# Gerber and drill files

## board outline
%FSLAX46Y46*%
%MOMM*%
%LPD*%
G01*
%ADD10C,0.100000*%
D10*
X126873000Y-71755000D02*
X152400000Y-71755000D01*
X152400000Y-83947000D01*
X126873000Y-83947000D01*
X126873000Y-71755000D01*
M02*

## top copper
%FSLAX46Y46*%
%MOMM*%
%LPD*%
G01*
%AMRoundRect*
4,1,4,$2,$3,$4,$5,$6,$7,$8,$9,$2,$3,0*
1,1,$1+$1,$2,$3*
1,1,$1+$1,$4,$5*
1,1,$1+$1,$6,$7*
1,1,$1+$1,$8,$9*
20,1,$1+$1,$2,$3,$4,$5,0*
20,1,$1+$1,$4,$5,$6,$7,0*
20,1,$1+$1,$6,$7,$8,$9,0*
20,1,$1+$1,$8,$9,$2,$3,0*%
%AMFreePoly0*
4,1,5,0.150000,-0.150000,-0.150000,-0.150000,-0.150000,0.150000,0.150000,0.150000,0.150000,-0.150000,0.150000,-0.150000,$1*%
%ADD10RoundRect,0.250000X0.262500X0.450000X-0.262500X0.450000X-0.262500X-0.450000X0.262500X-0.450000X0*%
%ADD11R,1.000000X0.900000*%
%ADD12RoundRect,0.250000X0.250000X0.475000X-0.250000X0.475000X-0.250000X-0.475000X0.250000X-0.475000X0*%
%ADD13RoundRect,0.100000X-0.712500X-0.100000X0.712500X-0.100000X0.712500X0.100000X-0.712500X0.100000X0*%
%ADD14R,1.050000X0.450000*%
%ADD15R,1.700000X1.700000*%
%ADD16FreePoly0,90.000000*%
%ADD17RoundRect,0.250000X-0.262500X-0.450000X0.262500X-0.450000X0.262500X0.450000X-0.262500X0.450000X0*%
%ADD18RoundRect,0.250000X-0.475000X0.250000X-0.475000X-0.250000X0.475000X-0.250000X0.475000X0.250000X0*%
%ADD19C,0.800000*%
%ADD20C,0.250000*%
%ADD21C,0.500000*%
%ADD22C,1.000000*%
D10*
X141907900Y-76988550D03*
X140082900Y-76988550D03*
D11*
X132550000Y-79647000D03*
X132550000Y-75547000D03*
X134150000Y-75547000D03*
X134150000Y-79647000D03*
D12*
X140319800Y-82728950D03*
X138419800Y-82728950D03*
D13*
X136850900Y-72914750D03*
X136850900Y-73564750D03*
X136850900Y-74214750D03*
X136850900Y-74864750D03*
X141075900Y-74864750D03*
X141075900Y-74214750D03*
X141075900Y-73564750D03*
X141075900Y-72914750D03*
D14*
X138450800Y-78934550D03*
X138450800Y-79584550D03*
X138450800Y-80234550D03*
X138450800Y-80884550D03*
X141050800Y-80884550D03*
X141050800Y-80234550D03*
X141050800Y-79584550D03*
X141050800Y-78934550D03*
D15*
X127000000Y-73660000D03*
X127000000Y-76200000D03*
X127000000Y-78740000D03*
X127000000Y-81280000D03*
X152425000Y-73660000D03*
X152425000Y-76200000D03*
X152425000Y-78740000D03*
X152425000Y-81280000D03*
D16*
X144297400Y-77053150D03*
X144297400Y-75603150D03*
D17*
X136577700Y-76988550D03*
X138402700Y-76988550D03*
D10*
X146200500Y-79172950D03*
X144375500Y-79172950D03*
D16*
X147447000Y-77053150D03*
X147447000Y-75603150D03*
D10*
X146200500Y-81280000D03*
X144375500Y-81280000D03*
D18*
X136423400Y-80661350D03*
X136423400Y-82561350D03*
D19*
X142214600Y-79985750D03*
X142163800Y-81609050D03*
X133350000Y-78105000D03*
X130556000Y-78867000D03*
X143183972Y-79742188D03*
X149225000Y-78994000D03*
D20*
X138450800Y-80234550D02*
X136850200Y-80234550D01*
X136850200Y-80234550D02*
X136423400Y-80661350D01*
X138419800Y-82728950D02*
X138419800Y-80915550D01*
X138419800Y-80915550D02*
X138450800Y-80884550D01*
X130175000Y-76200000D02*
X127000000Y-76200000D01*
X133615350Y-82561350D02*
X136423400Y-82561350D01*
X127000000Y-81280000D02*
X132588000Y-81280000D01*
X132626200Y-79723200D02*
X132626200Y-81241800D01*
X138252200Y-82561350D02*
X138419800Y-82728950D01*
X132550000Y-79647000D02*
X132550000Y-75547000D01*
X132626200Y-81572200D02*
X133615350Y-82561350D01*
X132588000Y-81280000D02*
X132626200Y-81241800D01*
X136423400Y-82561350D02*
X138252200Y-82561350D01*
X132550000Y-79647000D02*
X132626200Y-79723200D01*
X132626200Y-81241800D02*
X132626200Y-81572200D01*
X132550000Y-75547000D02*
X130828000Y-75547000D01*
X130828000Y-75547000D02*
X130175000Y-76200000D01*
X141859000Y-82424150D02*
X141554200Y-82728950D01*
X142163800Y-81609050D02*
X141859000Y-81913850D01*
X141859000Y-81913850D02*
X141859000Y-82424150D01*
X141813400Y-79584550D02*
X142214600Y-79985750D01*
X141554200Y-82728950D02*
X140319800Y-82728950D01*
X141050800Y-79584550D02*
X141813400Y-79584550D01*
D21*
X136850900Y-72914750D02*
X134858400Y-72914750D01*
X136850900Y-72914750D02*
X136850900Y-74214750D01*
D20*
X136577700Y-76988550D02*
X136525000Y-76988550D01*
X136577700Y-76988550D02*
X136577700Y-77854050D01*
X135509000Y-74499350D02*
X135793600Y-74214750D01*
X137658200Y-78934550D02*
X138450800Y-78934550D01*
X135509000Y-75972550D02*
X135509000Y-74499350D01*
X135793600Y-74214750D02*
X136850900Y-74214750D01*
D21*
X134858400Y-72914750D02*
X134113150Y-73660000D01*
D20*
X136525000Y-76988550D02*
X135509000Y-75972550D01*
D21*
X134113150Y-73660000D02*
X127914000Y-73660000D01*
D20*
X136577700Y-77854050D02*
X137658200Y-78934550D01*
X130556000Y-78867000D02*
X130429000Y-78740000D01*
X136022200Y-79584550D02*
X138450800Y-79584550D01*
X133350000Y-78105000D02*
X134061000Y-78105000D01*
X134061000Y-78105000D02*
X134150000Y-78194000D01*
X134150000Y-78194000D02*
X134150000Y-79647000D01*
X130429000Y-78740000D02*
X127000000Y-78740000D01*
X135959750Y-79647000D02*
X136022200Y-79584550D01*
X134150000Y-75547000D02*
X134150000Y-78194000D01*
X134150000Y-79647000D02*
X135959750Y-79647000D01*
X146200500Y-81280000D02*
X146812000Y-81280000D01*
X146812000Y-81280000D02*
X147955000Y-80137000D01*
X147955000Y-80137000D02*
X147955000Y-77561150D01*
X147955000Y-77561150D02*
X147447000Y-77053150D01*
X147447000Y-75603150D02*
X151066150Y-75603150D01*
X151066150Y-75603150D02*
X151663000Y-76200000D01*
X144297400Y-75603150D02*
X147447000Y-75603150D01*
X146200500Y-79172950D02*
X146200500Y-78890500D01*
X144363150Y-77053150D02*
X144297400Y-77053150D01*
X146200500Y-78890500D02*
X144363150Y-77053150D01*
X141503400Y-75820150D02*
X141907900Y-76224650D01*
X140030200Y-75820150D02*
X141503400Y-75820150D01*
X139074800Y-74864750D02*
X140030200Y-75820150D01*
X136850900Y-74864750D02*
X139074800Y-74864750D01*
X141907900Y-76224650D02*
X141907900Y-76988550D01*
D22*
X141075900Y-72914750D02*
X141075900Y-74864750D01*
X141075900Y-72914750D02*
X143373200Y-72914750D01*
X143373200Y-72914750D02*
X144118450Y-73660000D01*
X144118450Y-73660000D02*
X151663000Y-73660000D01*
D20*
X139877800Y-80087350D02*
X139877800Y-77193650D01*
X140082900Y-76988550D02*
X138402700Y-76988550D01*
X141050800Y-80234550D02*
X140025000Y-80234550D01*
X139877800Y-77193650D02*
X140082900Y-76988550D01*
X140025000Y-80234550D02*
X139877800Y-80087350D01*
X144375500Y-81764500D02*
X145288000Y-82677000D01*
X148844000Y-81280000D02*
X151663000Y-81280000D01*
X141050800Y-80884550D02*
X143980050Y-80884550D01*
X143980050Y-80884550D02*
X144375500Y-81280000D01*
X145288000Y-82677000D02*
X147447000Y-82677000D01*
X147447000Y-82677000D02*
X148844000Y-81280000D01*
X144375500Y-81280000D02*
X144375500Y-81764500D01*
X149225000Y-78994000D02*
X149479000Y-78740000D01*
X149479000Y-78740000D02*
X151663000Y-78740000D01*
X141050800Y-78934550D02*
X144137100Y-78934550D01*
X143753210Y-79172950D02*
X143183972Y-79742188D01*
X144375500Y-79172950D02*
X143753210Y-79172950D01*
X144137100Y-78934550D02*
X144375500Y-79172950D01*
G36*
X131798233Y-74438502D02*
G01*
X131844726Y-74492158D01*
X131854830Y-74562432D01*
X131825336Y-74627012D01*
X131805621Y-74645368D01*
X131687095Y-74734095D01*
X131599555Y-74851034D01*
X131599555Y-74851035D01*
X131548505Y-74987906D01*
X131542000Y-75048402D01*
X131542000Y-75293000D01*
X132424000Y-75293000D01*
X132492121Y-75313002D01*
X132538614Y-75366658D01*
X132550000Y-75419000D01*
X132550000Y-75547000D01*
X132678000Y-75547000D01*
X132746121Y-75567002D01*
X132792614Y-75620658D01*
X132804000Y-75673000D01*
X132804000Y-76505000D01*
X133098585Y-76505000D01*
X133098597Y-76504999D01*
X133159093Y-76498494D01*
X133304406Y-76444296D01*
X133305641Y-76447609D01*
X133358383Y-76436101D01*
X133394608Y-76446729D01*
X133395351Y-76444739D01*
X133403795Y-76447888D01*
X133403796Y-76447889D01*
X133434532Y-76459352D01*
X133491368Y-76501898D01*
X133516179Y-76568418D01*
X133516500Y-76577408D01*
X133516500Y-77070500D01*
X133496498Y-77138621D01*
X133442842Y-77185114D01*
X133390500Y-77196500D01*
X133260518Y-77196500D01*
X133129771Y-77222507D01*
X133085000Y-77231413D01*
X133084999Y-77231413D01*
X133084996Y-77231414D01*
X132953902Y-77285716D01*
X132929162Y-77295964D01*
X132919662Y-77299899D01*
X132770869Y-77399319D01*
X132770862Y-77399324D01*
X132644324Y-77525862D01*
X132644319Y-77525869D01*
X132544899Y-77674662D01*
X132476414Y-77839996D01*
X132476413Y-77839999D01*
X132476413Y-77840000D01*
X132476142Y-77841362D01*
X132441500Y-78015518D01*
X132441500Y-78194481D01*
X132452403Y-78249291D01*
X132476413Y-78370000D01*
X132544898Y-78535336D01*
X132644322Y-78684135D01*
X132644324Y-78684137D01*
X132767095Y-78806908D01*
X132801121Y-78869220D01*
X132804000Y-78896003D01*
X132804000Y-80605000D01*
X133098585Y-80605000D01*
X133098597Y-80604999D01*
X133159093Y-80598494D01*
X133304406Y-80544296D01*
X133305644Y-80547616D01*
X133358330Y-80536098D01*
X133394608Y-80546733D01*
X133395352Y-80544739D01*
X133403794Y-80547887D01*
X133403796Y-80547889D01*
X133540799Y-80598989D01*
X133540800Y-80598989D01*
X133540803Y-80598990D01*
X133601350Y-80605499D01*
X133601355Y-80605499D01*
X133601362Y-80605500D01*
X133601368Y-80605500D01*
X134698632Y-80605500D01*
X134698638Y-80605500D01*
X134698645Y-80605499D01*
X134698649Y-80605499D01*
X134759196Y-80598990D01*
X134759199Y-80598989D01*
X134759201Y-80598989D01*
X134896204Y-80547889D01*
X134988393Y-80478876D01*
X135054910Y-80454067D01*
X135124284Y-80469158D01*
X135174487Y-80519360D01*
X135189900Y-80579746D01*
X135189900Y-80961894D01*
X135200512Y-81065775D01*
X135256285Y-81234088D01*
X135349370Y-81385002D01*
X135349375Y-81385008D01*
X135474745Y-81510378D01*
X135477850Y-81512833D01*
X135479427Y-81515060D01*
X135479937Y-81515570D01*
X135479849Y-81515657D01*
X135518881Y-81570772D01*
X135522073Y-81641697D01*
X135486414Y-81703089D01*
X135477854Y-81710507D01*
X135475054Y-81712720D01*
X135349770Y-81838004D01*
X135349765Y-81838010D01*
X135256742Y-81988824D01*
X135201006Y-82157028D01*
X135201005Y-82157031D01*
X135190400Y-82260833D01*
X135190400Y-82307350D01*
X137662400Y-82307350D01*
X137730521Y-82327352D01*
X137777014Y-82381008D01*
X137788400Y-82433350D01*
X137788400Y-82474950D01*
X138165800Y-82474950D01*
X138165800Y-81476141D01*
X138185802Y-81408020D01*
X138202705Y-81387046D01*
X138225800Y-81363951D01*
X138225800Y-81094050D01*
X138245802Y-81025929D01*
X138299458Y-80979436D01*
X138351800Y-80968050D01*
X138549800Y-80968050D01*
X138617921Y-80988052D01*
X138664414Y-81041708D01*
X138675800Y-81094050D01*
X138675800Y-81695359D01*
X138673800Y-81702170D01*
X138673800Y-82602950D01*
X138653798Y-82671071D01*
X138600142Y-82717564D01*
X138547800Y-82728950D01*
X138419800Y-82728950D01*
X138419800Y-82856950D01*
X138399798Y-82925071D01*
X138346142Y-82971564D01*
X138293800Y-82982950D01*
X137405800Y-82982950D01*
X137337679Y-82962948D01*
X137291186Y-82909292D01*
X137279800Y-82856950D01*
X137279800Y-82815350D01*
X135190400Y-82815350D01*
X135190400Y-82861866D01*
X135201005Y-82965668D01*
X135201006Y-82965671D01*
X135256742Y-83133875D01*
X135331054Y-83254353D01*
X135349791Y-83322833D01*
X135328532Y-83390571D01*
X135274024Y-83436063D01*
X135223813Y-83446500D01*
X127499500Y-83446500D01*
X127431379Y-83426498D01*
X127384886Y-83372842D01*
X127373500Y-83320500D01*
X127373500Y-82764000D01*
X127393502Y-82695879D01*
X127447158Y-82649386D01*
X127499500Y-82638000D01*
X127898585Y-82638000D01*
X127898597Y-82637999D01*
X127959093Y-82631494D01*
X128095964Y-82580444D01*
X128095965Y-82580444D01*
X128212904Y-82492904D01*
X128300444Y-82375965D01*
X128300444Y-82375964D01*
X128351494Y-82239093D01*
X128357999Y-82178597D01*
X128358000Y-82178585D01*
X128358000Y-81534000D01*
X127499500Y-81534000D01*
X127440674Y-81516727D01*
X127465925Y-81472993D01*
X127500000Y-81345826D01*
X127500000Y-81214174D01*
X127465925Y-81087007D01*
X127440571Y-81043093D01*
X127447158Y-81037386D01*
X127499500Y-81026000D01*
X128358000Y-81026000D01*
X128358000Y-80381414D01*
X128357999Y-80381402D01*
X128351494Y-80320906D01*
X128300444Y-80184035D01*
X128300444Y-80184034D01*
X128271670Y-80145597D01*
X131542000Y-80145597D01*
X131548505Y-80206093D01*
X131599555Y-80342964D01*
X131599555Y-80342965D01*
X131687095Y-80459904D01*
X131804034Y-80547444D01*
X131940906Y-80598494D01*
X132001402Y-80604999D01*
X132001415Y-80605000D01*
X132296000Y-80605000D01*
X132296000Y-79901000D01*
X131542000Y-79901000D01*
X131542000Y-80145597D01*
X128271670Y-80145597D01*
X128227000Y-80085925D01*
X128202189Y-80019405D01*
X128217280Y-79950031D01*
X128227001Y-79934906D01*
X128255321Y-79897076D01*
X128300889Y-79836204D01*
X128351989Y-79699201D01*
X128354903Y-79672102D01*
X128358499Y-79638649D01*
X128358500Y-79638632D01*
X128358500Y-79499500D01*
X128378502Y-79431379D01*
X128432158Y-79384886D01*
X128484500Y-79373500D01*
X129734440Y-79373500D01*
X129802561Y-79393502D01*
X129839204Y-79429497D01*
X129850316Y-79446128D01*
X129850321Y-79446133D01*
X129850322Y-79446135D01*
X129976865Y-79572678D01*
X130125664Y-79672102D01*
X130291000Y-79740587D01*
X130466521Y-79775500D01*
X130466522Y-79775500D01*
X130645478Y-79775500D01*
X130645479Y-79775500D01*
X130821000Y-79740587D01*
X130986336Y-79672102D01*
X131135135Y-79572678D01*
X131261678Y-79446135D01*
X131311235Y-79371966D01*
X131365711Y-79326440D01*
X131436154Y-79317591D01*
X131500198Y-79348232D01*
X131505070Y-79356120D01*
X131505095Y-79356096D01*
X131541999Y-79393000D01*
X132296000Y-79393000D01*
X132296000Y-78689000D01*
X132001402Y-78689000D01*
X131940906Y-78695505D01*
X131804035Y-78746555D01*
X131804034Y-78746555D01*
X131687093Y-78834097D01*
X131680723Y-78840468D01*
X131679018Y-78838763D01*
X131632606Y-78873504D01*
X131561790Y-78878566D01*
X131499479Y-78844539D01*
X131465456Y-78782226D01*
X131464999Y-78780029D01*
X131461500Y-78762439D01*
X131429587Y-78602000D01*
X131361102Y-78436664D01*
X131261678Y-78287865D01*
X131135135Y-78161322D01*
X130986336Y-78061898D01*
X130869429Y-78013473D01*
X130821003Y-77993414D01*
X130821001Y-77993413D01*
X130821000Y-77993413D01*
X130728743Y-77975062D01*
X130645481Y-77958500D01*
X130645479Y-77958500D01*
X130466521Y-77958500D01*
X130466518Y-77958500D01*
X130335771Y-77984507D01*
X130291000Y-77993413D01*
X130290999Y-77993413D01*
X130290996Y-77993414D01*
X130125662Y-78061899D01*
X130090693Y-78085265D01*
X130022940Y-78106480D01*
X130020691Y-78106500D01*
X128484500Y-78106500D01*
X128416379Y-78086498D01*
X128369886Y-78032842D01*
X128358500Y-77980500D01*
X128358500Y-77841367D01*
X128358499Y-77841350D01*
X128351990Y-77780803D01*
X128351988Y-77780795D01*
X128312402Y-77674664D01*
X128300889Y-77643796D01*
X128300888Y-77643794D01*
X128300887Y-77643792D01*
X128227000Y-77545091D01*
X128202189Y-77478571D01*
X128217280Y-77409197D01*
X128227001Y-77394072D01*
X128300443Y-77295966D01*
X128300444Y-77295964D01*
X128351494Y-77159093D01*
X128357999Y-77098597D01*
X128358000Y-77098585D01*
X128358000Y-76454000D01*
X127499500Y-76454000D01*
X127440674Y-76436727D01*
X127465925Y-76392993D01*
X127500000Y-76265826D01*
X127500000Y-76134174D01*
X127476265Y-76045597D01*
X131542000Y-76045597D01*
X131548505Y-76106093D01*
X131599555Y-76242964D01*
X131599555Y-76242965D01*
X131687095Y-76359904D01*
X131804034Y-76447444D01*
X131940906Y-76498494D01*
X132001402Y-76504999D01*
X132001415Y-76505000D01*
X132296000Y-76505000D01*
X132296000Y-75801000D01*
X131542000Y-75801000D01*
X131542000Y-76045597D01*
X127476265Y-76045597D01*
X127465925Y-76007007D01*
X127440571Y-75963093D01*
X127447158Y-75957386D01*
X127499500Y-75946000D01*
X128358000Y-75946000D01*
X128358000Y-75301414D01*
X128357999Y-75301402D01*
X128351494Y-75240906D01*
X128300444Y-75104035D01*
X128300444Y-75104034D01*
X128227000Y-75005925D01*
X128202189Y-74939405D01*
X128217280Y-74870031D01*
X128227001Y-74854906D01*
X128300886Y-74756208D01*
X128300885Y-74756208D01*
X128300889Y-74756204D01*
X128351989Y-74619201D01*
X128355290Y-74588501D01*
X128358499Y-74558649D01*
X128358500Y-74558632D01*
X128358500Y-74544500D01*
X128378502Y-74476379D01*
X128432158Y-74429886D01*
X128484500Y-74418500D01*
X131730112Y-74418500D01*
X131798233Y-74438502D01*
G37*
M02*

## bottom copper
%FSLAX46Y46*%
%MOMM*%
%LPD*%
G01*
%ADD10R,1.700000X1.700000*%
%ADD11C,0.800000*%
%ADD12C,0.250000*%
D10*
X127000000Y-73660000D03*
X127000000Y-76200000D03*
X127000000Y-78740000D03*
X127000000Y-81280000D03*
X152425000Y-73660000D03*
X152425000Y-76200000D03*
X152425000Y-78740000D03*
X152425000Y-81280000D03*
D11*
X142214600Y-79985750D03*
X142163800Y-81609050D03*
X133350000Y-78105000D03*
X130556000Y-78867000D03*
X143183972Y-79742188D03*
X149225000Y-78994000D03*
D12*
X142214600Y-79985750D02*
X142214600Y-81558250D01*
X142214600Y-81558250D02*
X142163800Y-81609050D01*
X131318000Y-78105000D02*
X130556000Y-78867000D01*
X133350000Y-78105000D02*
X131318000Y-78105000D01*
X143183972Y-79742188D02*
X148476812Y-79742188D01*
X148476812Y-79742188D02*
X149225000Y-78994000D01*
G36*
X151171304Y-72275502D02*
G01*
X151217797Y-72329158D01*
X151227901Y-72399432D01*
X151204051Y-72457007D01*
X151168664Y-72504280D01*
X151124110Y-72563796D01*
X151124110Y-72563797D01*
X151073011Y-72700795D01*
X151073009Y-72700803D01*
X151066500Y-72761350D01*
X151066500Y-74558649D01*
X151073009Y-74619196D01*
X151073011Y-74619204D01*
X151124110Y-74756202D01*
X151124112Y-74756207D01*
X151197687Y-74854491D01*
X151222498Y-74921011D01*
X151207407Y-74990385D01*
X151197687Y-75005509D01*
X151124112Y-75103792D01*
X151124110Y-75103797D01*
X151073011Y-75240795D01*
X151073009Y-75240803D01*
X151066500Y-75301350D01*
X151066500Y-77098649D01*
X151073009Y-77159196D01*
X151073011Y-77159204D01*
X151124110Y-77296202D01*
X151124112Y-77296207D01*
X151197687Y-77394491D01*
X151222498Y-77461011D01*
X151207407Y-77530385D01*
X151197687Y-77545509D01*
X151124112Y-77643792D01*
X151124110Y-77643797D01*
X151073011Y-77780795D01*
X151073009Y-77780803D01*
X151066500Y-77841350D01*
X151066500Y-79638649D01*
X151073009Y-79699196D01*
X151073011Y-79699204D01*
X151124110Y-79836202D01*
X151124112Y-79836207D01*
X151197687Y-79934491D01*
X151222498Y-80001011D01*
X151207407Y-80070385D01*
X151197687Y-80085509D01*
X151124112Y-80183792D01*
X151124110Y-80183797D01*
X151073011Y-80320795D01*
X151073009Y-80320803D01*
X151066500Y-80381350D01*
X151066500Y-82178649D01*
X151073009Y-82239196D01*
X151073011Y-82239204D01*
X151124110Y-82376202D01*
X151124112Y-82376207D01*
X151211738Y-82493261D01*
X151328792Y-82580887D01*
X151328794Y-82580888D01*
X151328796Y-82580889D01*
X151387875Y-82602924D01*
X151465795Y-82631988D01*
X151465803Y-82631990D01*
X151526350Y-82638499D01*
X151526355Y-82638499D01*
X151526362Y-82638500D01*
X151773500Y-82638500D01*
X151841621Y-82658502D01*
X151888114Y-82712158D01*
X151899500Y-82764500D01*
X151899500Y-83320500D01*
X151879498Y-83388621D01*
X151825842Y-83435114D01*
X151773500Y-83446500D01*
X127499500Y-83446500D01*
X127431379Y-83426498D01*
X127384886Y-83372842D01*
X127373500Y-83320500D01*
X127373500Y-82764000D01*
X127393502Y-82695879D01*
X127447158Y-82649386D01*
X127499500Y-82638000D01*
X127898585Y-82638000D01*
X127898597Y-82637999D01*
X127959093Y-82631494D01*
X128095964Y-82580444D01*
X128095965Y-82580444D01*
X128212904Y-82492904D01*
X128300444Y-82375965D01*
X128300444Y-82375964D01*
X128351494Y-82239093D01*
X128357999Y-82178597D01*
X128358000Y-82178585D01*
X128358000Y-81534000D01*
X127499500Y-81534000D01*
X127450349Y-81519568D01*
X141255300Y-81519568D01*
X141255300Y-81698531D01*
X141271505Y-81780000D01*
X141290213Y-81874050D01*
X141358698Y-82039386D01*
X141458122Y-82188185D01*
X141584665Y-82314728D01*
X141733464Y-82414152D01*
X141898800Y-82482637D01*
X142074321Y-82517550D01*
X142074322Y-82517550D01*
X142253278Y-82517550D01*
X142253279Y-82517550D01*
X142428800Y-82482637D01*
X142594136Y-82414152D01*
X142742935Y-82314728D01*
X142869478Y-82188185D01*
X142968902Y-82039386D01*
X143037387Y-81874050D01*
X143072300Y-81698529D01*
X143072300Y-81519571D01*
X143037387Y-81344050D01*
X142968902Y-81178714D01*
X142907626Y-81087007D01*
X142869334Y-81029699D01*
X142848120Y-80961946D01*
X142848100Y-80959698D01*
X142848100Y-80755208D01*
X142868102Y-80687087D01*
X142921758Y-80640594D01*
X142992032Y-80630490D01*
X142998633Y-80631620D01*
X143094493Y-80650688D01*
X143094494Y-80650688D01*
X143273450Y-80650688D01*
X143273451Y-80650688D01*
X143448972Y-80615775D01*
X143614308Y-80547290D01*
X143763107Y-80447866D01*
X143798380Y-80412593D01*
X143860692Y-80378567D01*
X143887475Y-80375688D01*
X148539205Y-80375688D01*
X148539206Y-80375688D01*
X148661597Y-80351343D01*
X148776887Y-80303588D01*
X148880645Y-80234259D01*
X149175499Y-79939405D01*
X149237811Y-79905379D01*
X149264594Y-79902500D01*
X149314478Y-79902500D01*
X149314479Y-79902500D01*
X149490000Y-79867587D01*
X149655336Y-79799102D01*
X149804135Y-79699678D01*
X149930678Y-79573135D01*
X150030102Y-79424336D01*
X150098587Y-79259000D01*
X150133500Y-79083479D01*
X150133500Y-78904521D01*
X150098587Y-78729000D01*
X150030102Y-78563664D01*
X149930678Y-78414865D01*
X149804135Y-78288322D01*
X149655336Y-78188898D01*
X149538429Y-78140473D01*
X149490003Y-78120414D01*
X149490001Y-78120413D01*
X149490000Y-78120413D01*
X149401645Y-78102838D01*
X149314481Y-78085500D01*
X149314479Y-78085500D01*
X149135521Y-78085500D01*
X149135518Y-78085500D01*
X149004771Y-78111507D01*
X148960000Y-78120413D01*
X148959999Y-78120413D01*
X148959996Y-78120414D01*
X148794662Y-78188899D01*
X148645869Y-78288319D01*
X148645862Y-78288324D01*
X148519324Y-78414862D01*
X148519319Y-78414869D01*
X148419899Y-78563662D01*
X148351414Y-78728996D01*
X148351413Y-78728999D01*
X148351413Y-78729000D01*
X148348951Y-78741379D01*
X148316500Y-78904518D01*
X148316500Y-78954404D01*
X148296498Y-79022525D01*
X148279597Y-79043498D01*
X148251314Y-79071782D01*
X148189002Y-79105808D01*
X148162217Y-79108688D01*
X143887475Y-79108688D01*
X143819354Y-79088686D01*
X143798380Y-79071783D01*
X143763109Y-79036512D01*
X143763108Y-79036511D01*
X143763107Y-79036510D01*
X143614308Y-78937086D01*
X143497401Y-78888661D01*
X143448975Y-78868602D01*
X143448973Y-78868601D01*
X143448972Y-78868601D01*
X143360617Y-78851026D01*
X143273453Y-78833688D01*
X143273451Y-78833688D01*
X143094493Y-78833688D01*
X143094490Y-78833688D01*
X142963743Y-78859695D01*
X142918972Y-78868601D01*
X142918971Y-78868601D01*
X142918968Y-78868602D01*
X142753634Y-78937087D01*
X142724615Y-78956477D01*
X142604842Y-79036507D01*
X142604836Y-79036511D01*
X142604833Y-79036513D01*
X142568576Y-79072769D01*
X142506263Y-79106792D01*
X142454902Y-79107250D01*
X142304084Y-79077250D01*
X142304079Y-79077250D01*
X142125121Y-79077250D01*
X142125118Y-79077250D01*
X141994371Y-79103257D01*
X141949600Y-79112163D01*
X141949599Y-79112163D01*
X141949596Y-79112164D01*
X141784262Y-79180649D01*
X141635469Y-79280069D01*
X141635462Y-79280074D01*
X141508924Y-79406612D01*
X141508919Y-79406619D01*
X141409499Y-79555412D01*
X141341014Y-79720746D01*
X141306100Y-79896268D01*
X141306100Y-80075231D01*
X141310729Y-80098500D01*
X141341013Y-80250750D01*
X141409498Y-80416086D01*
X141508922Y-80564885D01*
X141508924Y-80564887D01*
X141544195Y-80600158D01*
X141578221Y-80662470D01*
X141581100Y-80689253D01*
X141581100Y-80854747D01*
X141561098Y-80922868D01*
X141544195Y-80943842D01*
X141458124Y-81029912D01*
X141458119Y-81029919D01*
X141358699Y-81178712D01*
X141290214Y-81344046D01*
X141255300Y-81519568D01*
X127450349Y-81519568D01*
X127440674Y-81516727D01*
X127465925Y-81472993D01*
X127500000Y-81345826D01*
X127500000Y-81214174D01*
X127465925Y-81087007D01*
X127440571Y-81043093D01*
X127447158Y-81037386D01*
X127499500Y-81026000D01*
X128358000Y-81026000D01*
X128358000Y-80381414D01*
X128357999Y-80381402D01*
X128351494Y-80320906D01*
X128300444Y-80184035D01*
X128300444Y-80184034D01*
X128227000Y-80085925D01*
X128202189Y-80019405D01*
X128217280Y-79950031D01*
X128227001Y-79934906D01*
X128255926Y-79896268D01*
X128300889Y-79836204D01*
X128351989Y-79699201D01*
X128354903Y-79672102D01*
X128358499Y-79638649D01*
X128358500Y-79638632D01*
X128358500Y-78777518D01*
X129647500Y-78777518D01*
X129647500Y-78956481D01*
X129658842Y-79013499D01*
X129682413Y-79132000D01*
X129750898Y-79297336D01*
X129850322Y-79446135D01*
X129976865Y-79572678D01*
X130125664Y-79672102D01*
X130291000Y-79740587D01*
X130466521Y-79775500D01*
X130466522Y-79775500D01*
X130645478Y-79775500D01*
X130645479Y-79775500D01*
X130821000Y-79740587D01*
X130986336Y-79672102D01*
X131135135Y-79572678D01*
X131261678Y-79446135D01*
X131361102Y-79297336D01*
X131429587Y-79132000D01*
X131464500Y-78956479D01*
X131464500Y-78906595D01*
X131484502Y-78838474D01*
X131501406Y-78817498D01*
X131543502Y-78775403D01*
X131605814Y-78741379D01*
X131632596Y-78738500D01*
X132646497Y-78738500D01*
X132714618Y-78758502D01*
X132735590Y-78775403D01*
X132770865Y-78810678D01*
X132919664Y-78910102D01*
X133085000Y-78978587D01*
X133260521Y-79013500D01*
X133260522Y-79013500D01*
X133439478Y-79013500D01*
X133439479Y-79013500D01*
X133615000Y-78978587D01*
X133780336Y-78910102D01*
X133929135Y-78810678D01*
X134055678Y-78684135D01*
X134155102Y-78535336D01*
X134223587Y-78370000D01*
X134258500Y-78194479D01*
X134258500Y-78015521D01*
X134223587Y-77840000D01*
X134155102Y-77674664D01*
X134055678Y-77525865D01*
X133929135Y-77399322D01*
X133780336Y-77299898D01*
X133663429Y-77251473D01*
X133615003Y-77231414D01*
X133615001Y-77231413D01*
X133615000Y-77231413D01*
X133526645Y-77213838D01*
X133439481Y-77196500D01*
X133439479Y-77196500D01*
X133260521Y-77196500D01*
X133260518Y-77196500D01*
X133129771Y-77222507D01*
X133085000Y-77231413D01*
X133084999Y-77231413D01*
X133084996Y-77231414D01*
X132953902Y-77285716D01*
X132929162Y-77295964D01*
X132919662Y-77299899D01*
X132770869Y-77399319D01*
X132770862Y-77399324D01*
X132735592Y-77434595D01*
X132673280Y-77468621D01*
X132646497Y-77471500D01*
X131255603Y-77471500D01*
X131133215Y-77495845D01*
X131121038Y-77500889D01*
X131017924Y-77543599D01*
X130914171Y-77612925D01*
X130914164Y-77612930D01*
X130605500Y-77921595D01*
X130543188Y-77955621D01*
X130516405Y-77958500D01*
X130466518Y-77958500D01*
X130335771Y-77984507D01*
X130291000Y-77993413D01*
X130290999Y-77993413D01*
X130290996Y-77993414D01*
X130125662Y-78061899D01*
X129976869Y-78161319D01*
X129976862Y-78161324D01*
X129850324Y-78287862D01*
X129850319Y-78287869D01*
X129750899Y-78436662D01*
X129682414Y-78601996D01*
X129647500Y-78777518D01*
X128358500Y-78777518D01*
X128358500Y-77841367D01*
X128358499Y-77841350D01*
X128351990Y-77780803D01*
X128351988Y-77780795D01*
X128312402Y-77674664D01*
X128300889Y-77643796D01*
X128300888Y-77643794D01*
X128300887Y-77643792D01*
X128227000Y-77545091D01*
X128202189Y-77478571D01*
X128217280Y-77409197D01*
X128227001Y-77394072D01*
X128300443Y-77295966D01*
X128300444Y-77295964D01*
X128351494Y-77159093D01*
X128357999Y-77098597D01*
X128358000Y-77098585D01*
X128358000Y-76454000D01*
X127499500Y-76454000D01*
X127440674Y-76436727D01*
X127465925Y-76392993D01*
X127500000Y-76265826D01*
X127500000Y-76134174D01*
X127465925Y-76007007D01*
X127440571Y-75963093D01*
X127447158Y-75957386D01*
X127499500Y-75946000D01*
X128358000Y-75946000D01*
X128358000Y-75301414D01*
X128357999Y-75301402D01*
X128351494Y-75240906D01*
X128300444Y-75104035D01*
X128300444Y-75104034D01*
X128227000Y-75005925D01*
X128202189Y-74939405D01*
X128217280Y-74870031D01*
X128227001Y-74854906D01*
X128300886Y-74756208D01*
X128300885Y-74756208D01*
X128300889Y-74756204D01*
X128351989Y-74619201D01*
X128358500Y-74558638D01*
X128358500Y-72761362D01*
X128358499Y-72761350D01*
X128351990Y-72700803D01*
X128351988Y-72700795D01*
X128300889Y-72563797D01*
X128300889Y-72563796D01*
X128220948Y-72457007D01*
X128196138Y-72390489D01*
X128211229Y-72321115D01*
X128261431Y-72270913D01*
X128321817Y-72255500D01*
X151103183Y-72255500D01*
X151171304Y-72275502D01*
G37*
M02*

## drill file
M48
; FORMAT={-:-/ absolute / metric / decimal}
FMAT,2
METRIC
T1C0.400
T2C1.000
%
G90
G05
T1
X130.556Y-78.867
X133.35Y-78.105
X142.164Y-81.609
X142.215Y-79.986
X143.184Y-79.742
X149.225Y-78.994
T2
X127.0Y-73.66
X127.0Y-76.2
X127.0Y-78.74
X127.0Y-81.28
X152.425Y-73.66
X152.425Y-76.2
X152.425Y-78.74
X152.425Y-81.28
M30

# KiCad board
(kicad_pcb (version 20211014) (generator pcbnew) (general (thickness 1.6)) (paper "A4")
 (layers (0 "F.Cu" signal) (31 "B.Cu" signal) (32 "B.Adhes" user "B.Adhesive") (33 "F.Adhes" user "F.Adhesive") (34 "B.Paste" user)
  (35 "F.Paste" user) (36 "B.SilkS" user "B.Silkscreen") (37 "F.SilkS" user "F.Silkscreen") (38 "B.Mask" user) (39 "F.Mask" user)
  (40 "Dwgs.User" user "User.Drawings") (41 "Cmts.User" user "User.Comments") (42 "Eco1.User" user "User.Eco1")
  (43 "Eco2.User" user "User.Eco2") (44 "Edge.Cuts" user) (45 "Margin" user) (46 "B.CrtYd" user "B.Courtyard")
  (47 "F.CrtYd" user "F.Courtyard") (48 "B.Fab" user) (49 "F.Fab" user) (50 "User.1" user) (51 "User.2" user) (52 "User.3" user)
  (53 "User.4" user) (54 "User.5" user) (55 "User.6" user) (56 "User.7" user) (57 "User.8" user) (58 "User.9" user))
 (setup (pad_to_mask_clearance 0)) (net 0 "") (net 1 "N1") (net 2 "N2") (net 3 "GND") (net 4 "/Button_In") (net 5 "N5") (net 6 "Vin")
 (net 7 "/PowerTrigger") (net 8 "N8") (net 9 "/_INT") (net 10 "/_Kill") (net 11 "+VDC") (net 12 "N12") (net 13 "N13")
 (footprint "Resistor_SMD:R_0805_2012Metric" (layer "F.Cu") (at 140.9954 76.98855 180)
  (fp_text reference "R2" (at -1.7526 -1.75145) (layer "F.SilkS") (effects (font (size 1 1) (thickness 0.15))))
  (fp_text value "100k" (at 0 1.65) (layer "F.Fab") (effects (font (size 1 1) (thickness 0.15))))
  (pad "1" smd roundrect locked (at -0.9125 0 180) (size 1.025 1.4) (layers "F.Cu" "F.Paste" "F.Mask") (roundrect_rratio 0.243902)
   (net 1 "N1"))
  (pad "2" smd roundrect locked (at 0.9125 0 180) (size 1.025 1.4) (layers "F.Cu" "F.Paste" "F.Mask") (roundrect_rratio 0.243902)
   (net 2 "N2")))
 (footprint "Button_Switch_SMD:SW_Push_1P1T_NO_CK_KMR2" (layer "F.Cu") (at 133.35 77.597 90)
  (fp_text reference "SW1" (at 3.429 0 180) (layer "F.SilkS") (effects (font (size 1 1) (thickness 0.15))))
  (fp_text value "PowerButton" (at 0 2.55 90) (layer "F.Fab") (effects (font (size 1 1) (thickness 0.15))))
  (pad "1" smd rect locked (at -2.05 -0.8 90) (size 0.9 1) (layers "F.Cu" "F.Paste" "F.Mask") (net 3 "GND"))
  (pad "1" smd rect locked (at 2.05 -0.8 90) (size 0.9 1) (layers "F.Cu" "F.Paste" "F.Mask") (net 3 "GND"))
  (pad "2" smd rect locked (at 2.05 0.8 90) (size 0.9 1) (layers "F.Cu" "F.Paste" "F.Mask") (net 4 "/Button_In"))
  (pad "2" smd rect locked (at -2.05 0.8 90) (size 0.9 1) (layers "F.Cu" "F.Paste" "F.Mask") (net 4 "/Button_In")))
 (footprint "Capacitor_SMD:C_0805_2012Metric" (layer "F.Cu") (at 139.3698 82.72895 180)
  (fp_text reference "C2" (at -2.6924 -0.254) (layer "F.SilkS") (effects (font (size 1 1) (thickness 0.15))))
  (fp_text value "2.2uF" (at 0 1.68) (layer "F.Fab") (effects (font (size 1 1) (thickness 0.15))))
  (pad "1" smd roundrect locked (at -0.95 0 180) (size 1 1.45) (layers "F.Cu" "F.Paste" "F.Mask") (roundrect_rratio 0.25) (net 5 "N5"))
  (pad "2" smd roundrect locked (at 0.95 0 180) (size 1 1.45) (layers "F.Cu" "F.Paste" "F.Mask") (roundrect_rratio 0.25) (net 3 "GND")))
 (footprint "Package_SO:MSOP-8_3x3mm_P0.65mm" (layer "F.Cu") (at 138.9634 73.88975)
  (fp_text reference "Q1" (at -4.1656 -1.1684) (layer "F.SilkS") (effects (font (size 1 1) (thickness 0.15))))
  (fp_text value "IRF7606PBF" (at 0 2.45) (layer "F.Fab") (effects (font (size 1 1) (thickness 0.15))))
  (pad "1" smd roundrect locked (at -2.1125 -0.975) (size 1.625 0.4) (layers "F.Cu" "F.Paste" "F.Mask") (roundrect_rratio 0.25)
   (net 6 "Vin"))
  (pad "2" smd roundrect locked (at -2.1125 -0.325) (size 1.625 0.4) (layers "F.Cu" "F.Paste" "F.Mask") (roundrect_rratio 0.25)
   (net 6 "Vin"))
  (pad "3" smd roundrect locked (at -2.1125 0.325) (size 1.625 0.4) (layers "F.Cu" "F.Paste" "F.Mask") (roundrect_rratio 0.25) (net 6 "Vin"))
  (pad "4" smd roundrect locked (at -2.1125 0.975) (size 1.625 0.4) (layers "F.Cu" "F.Paste" "F.Mask") (roundrect_rratio 0.25) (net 1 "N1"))
  (pad "5" smd roundrect locked (at 2.1125 0.975) (size 1.625 0.4) (layers "F.Cu" "F.Paste" "F.Mask") (roundrect_rratio 0.25)
   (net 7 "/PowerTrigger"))
  (pad "6" smd roundrect locked (at 2.1125 0.325) (size 1.625 0.4) (layers "F.Cu" "F.Paste" "F.Mask") (roundrect_rratio 0.25)
   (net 7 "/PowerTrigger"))
  (pad "7" smd roundrect locked (at 2.1125 -0.325) (size 1.625 0.4) (layers "F.Cu" "F.Paste" "F.Mask") (roundrect_rratio 0.25)
   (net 7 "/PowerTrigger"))
  (pad "8" smd roundrect locked (at 2.1125 -0.975) (size 1.625 0.4) (layers "F.Cu" "F.Paste" "F.Mask") (roundrect_rratio 0.25)
   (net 7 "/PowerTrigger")))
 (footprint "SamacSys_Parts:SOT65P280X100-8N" (layer "F.Cu") (at 139.7508 79.90955)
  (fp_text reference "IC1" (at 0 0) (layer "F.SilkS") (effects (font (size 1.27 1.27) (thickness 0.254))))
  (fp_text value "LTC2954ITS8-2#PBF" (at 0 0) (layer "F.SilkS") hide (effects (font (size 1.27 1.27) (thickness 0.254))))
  (pad "1" smd rect locked (at -1.3 -0.975 90) (size 0.45 1.05) (layers "F.Cu" "F.Paste" "F.Mask") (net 6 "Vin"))
  (pad "2" smd rect locked (at -1.3 -0.325 90) (size 0.45 1.05) (layers "F.Cu" "F.Paste" "F.Mask") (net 4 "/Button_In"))
  (pad "3" smd rect locked (at -1.3 0.325 90) (size 0.45 1.05) (layers "F.Cu" "F.Paste" "F.Mask") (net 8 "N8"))
  (pad "4" smd rect locked (at -1.3 0.975 90) (size 0.45 1.05) (layers "F.Cu" "F.Paste" "F.Mask") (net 3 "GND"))
  (pad "5" smd rect locked (at 1.3 0.975 90) (size 0.45 1.05) (layers "F.Cu" "F.Paste" "F.Mask") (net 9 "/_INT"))
  (pad "6" smd rect locked (at 1.3 0.325 90) (size 0.45 1.05) (layers "F.Cu" "F.Paste" "F.Mask") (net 2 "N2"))
  (pad "7" smd rect locked (at 1.3 -0.325 90) (size 0.45 1.05) (layers "F.Cu" "F.Paste" "F.Mask") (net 5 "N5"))
  (pad "8" smd rect locked (at 1.3 -0.975 90) (size 0.45 1.05) (layers "F.Cu" "F.Paste" "F.Mask") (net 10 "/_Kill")))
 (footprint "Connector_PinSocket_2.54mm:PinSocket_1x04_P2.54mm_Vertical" (layer "F.Cu") (at 127 73.66)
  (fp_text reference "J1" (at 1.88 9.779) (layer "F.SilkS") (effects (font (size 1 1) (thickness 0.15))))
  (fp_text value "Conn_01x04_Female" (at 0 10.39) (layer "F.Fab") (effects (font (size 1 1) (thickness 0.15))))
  (pad "1" thru_hole rect locked (at 0 0) (size 1.7 1.7) (drill 1) (layers *.Cu *.Mask) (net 6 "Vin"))
  (pad "2" thru_hole rect locked (at 0 2.54) (size 1.7 1.7) (drill 1) (layers *.Cu *.Mask) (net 3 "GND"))
  (pad "3" thru_hole rect locked (at 0 5.08) (size 1.7 1.7) (drill 1) (layers *.Cu *.Mask) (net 4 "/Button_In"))
  (pad "4" thru_hole rect locked (at 0 7.62) (size 1.7 1.7) (drill 1) (layers *.Cu *.Mask) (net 3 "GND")))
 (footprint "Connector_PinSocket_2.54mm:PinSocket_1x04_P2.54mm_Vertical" (layer "F.Cu") (at 152.425 73.66)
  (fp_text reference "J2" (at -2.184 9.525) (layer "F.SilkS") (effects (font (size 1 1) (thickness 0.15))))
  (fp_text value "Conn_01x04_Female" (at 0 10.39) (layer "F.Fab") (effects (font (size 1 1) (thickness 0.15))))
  (pad "1" thru_hole rect locked (at 0 0) (size 1.7 1.7) (drill 1) (layers *.Cu *.Mask) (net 7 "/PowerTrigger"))
  (pad "2" thru_hole rect locked (at 0 2.54) (size 1.7 1.7) (drill 1) (layers *.Cu *.Mask) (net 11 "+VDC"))
  (pad "3" thru_hole rect locked (at 0 5.08) (size 1.7 1.7) (drill 1) (layers *.Cu *.Mask) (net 10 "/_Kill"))
  (pad "4" thru_hole rect locked (at 0 7.62) (size 1.7 1.7) (drill 1) (layers *.Cu *.Mask) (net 9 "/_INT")))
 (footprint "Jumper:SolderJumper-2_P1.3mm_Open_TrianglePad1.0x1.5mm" (layer "F.Cu") (at 144.2974 76.32815 90)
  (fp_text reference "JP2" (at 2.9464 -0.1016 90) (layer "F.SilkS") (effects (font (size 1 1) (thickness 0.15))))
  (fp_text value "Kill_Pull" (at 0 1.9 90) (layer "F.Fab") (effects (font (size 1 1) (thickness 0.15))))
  (pad "1" smd custom locked (at -0.725 0 90) (size 0.3 0.3) (layers "F.Cu" "F.Mask") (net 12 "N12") (zone_connect 2)
   (options (clearance outline) (anchor rect)) (primitives))
  (pad "2" smd custom locked (at 0.725 0 90) (size 0.3 0.3) (layers "F.Cu" "F.Mask") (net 11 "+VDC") (zone_connect 2)
   (options (clearance outline) (anchor rect)) (primitives)))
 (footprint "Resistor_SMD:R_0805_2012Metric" (layer "F.Cu") (at 137.4902 76.98855)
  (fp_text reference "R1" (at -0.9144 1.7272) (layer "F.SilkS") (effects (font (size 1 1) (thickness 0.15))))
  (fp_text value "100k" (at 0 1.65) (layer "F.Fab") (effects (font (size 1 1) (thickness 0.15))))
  (pad "1" smd roundrect locked (at -0.9125 0) (size 1.025 1.4) (layers "F.Cu" "F.Paste" "F.Mask") (roundrect_rratio 0.243902) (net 6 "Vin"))
  (pad "2" smd roundrect locked (at 0.9125 0) (size 1.025 1.4) (layers "F.Cu" "F.Paste" "F.Mask") (roundrect_rratio 0.243902) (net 2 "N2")))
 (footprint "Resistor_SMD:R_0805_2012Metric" (layer "F.Cu") (at 145.288 79.17295 180)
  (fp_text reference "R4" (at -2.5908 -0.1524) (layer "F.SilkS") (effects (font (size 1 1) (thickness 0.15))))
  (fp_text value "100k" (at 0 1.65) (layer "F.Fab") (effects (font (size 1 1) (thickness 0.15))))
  (pad "1" smd roundrect locked (at -0.9125 0 180) (size 1.025 1.4) (layers "F.Cu" "F.Paste" "F.Mask") (roundrect_rratio 0.243902)
   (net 12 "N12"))
  (pad "2" smd roundrect locked (at 0.9125 0 180) (size 1.025 1.4) (layers "F.Cu" "F.Paste" "F.Mask") (roundrect_rratio 0.243902)
   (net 10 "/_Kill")))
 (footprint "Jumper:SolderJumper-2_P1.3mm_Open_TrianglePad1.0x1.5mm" (layer "F.Cu") (at 147.447 76.32815 90)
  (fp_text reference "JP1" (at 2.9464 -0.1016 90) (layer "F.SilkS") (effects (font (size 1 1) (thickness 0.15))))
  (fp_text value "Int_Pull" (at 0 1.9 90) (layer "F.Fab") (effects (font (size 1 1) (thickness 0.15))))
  (pad "1" smd custom locked (at -0.725 0 90) (size 0.3 0.3) (layers "F.Cu" "F.Mask") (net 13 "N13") (zone_connect 2)
   (options (clearance outline) (anchor rect)) (primitives))
  (pad "2" smd custom locked (at 0.725 0 90) (size 0.3 0.3) (layers "F.Cu" "F.Mask") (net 11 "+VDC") (zone_connect 2)
   (options (clearance outline) (anchor rect)) (primitives)))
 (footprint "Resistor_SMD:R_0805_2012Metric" (layer "F.Cu") (at 145.288 81.28 180)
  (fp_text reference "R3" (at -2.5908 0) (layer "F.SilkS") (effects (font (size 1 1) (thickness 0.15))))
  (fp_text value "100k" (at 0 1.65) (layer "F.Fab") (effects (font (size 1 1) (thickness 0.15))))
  (pad "1" smd roundrect locked (at -0.9125 0 180) (size 1.025 1.4) (layers "F.Cu" "F.Paste" "F.Mask") (roundrect_rratio 0.243902)
   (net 13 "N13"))
  (pad "2" smd roundrect locked (at 0.9125 0 180) (size 1.025 1.4) (layers "F.Cu" "F.Paste" "F.Mask") (roundrect_rratio 0.243902)
   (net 9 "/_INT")))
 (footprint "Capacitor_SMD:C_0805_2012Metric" (layer "F.Cu") (at 136.4234 81.61135 -90)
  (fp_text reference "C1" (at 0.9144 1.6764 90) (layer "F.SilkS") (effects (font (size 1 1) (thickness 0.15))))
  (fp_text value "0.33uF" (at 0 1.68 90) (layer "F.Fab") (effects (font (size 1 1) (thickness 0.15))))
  (pad "1" smd roundrect locked (at -0.95 0 270) (size 1 1.45) (layers "F.Cu" "F.Paste" "F.Mask") (roundrect_rratio 0.25) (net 8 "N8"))
  (pad "2" smd roundrect locked (at 0.95 0 270) (size 1 1.45) (layers "F.Cu" "F.Paste" "F.Mask") (roundrect_rratio 0.25) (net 3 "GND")))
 (gr_rect (start 126.873 71.755) (end 152.4 83.947) (layer "Edge.Cuts") (width 0.1) (fill none))
 (segment (start 138.4508 80.23455) (end 136.8502 80.23455) (width 0.25) (layer "F.Cu") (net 8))
 (segment (start 136.8502 80.23455) (end 136.4234 80.66135) (width 0.25) (layer "F.Cu") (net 8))
 (segment (start 138.4198 82.72895) (end 138.4198 80.91555) (width 0.25) (layer "F.Cu") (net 3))
 (segment (start 138.4198 80.91555) (end 138.4508 80.88455) (width 0.25) (layer "F.Cu") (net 3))
 (segment (start 130.175 76.2) (end 127 76.2) (width 0.25) (layer "F.Cu") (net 3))
 (segment (start 133.61535 82.56135) (end 136.4234 82.56135) (width 0.25) (layer "F.Cu") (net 3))
 (segment (start 127 81.28) (end 132.588 81.28) (width 0.25) (layer "F.Cu") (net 3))
 (segment (start 132.6262 79.7232) (end 132.6262 81.2418) (width 0.25) (layer "F.Cu") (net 3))
 (segment (start 138.2522 82.56135) (end 138.4198 82.72895) (width 0.25) (layer "F.Cu") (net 3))
 (segment (start 132.55 79.647) (end 132.55 75.547) (width 0.25) (layer "F.Cu") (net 3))
 (segment (start 132.6262 81.5722) (end 133.61535 82.56135) (width 0.25) (layer "F.Cu") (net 3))
 (segment (start 132.588 81.28) (end 132.6262 81.2418) (width 0.25) (layer "F.Cu") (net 3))
 (segment (start 136.4234 82.56135) (end 138.2522 82.56135) (width 0.25) (layer "F.Cu") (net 3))
 (segment (start 132.55 79.647) (end 132.6262 79.7232) (width 0.25) (layer "F.Cu") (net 3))
 (segment (start 132.6262 81.2418) (end 132.6262 81.5722) (width 0.25) (layer "F.Cu") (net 3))
 (segment (start 132.55 75.547) (end 130.828 75.547) (width 0.25) (layer "F.Cu") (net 3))
 (segment (start 130.828 75.547) (end 130.175 76.2) (width 0.25) (layer "F.Cu") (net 3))
 (segment (start 141.859 82.42415) (end 141.5542 82.72895) (width 0.25) (layer "F.Cu") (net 5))
 (segment (start 142.1638 81.60905) (end 141.859 81.91385) (width 0.25) (layer "F.Cu") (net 5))
 (segment (start 141.859 81.91385) (end 141.859 82.42415) (width 0.25) (layer "F.Cu") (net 5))
 (segment (start 141.8134 79.58455) (end 142.2146 79.98575) (width 0.25) (layer "F.Cu") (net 5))
 (segment (start 141.5542 82.72895) (end 140.3198 82.72895) (width 0.25) (layer "F.Cu") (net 5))
 (segment (start 141.0508 79.58455) (end 141.8134 79.58455) (width 0.25) (layer "F.Cu") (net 5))
 (via (at 142.2146 79.98575) (size 0.8) (drill 0.4) (layers "F.Cu" "B.Cu") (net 5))
 (via (at 142.1638 81.60905) (size 0.8) (drill 0.4) (layers "F.Cu" "B.Cu") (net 5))
 (segment (start 142.2146 79.98575) (end 142.2146 81.55825) (width 0.25) (layer "B.Cu") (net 5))
 (segment (start 142.2146 81.55825) (end 142.1638 81.60905) (width 0.25) (layer "B.Cu") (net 5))
 (segment (start 136.8509 72.91475) (end 134.8584 72.91475) (width 0.5) (layer "F.Cu") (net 6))
 (segment (start 136.8509 72.91475) (end 136.8509 74.21475) (width 0.5) (layer "F.Cu") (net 6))
 (segment (start 136.5777 76.98855) (end 136.525 76.98855) (width 0.25) (layer "F.Cu") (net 6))
 (segment (start 136.5777 76.98855) (end 136.5777 77.85405) (width 0.25) (layer "F.Cu") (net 6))
 (segment (start 135.509 74.49935) (end 135.7936 74.21475) (width 0.25) (layer "F.Cu") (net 6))
 (segment (start 137.6582 78.93455) (end 138.4508 78.93455) (width 0.25) (layer "F.Cu") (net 6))
 (segment (start 135.509 75.97255) (end 135.509 74.49935) (width 0.25) (layer "F.Cu") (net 6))
 (segment (start 135.7936 74.21475) (end 136.8509 74.21475) (width 0.25) (layer "F.Cu") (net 6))
 (segment (start 134.8584 72.91475) (end 134.11315 73.66) (width 0.5) (layer "F.Cu") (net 6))
 (segment (start 136.525 76.98855) (end 135.509 75.97255) (width 0.25) (layer "F.Cu") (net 6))
 (segment (start 134.11315 73.66) (end 127.914 73.66) (width 0.5) (layer "F.Cu") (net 6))
 (segment (start 136.5777 77.85405) (end 137.6582 78.93455) (width 0.25) (layer "F.Cu") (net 6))
 (segment (start 130.556 78.867) (end 130.429 78.74) (width 0.25) (layer "F.Cu") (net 4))
 (segment (start 136.0222 79.58455) (end 138.4508 79.58455) (width 0.25) (layer "F.Cu") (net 4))
 (segment (start 133.35 78.105) (end 134.061 78.105) (width 0.25) (layer "F.Cu") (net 4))
 (segment (start 134.061 78.105) (end 134.15 78.194) (width 0.25) (layer "F.Cu") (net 4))
 (segment (start 134.15 78.194) (end 134.15 79.647) (width 0.25) (layer "F.Cu") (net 4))
 (segment (start 130.429 78.74) (end 127 78.74) (width 0.25) (layer "F.Cu") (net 4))
 (segment (start 135.95975 79.647) (end 136.0222 79.58455) (width 0.25) (layer "F.Cu") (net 4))
 (segment (start 134.15 75.547) (end 134.15 78.194) (width 0.25) (layer "F.Cu") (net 4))
 (segment (start 134.15 79.647) (end 135.95975 79.647) (width 0.25) (layer "F.Cu") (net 4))
 (via (at 133.35 78.105) (size 0.8) (drill 0.4) (layers "F.Cu" "B.Cu") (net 4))
 (via (at 130.556 78.867) (size 0.8) (drill 0.4) (layers "F.Cu" "B.Cu") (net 4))
 (segment (start 131.318 78.105) (end 130.556 78.867) (width 0.25) (layer "B.Cu") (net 4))
 (segment (start 133.35 78.105) (end 131.318 78.105) (width 0.25) (layer "B.Cu") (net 4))
 (segment (start 146.2005 81.28) (end 146.812 81.28) (width 0.25) (layer "F.Cu") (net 13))
 (segment (start 146.812 81.28) (end 147.955 80.137) (width 0.25) (layer "F.Cu") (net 13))
 (segment (start 147.955 80.137) (end 147.955 77.56115) (width 0.25) (layer "F.Cu") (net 13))
 (segment (start 147.955 77.56115) (end 147.447 77.05315) (width 0.25) (layer "F.Cu") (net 13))
 (segment (start 147.447 75.60315) (end 151.06615 75.60315) (width 0.25) (layer "F.Cu") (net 11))
 (segment (start 151.06615 75.60315) (end 151.663 76.2) (width 0.25) (layer "F.Cu") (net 11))
 (segment (start 144.2974 75.60315) (end 147.447 75.60315) (width 0.25) (layer "F.Cu") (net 11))
 (segment (start 146.2005 79.17295) (end 146.2005 78.8905) (width 0.25) (layer "F.Cu") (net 12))
 (segment (start 144.36315 77.05315) (end 144.2974 77.05315) (width 0.25) (layer "F.Cu") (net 12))
 (segment (start 146.2005 78.8905) (end 144.36315 77.05315) (width 0.25) (layer "F.Cu") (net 12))
 (segment (start 141.5034 75.82015) (end 141.9079 76.22465) (width 0.25) (layer "F.Cu") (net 1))
 (segment (start 140.0302 75.82015) (end 141.5034 75.82015) (width 0.25) (layer "F.Cu") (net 1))
 (segment (start 139.0748 74.86475) (end 140.0302 75.82015) (width 0.25) (layer "F.Cu") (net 1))
 (segment (start 136.8509 74.86475) (end 139.0748 74.86475) (width 0.25) (layer "F.Cu") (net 1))
 (segment (start 141.9079 76.22465) (end 141.9079 76.98855) (width 0.25) (layer "F.Cu") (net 1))
 (segment (start 141.0759 72.91475) (end 141.0759 74.86475) (width 1) (layer "F.Cu") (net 7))
 (segment (start 141.0759 72.91475) (end 143.3732 72.91475) (width 1) (layer "F.Cu") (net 7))
 (segment (start 143.3732 72.91475) (end 144.11845 73.66) (width 1) (layer "F.Cu") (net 7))
 (segment (start 144.11845 73.66) (end 151.663 73.66) (width 1) (layer "F.Cu") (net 7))
 (segment (start 139.8778 80.08735) (end 139.8778 77.19365) (width 0.25) (layer "F.Cu") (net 2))
 (segment (start 140.0829 76.98855) (end 138.4027 76.98855) (width 0.25) (layer "F.Cu") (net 2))
 (segment (start 141.0508 80.23455) (end 140.025 80.23455) (width 0.25) (layer "F.Cu") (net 2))
 (segment (start 139.8778 77.19365) (end 140.0829 76.98855) (width 0.25) (layer "F.Cu") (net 2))
 (segment (start 140.025 80.23455) (end 139.8778 80.08735) (width 0.25) (layer "F.Cu") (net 2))
 (segment (start 144.3755 81.7645) (end 145.288 82.677) (width 0.25) (layer "F.Cu") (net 9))
 (segment (start 148.844 81.28) (end 151.663 81.28) (width 0.25) (layer "F.Cu") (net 9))
 (segment (start 141.0508 80.88455) (end 143.98005 80.88455) (width 0.25) (layer "F.Cu") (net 9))
 (segment (start 143.98005 80.88455) (end 144.3755 81.28) (width 0.25) (layer "F.Cu") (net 9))
 (segment (start 145.288 82.677) (end 147.447 82.677) (width 0.25) (layer "F.Cu") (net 9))
 (segment (start 147.447 82.677) (end 148.844 81.28) (width 0.25) (layer "F.Cu") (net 9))
 (segment (start 144.3755 81.28) (end 144.3755 81.7645) (width 0.25) (layer "F.Cu") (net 9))
 (segment (start 149.225 78.994) (end 149.479 78.74) (width 0.25) (layer "F.Cu") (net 10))
 (segment (start 149.479 78.74) (end 151.663 78.74) (width 0.25) (layer "F.Cu") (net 10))
 (segment (start 141.0508 78.93455) (end 144.1371 78.93455) (width 0.25) (layer "F.Cu") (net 10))
 (segment (start 143.75321 79.17295) (end 143.183972 79.742188) (width 0.25) (layer "F.Cu") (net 10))
 (segment (start 144.3755 79.17295) (end 143.75321 79.17295) (width 0.25) (layer "F.Cu") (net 10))
 (segment (start 144.1371 78.93455) (end 144.3755 79.17295) (width 0.25) (layer "F.Cu") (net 10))
 (via (at 143.183972 79.742188) (size 0.8) (drill 0.4) (layers "F.Cu" "B.Cu") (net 10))
 (via (at 149.225 78.994) (size 0.8) (drill 0.4) (layers "F.Cu" "B.Cu") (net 10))
 (segment (start 143.183972 79.742188) (end 148.476812 79.742188) (width 0.25) (layer "B.Cu") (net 10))
 (segment (start 148.476812 79.742188) (end 149.225 78.994) (width 0.25) (layer "B.Cu") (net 10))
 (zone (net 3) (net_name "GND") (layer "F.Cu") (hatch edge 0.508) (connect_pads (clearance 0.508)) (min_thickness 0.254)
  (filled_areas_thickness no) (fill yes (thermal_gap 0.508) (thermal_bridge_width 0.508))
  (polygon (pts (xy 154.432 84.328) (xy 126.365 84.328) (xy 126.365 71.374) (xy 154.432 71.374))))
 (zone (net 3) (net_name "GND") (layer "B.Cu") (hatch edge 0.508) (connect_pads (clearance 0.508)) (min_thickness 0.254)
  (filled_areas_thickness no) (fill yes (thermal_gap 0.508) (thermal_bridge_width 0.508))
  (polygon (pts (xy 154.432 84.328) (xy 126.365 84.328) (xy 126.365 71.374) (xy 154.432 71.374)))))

